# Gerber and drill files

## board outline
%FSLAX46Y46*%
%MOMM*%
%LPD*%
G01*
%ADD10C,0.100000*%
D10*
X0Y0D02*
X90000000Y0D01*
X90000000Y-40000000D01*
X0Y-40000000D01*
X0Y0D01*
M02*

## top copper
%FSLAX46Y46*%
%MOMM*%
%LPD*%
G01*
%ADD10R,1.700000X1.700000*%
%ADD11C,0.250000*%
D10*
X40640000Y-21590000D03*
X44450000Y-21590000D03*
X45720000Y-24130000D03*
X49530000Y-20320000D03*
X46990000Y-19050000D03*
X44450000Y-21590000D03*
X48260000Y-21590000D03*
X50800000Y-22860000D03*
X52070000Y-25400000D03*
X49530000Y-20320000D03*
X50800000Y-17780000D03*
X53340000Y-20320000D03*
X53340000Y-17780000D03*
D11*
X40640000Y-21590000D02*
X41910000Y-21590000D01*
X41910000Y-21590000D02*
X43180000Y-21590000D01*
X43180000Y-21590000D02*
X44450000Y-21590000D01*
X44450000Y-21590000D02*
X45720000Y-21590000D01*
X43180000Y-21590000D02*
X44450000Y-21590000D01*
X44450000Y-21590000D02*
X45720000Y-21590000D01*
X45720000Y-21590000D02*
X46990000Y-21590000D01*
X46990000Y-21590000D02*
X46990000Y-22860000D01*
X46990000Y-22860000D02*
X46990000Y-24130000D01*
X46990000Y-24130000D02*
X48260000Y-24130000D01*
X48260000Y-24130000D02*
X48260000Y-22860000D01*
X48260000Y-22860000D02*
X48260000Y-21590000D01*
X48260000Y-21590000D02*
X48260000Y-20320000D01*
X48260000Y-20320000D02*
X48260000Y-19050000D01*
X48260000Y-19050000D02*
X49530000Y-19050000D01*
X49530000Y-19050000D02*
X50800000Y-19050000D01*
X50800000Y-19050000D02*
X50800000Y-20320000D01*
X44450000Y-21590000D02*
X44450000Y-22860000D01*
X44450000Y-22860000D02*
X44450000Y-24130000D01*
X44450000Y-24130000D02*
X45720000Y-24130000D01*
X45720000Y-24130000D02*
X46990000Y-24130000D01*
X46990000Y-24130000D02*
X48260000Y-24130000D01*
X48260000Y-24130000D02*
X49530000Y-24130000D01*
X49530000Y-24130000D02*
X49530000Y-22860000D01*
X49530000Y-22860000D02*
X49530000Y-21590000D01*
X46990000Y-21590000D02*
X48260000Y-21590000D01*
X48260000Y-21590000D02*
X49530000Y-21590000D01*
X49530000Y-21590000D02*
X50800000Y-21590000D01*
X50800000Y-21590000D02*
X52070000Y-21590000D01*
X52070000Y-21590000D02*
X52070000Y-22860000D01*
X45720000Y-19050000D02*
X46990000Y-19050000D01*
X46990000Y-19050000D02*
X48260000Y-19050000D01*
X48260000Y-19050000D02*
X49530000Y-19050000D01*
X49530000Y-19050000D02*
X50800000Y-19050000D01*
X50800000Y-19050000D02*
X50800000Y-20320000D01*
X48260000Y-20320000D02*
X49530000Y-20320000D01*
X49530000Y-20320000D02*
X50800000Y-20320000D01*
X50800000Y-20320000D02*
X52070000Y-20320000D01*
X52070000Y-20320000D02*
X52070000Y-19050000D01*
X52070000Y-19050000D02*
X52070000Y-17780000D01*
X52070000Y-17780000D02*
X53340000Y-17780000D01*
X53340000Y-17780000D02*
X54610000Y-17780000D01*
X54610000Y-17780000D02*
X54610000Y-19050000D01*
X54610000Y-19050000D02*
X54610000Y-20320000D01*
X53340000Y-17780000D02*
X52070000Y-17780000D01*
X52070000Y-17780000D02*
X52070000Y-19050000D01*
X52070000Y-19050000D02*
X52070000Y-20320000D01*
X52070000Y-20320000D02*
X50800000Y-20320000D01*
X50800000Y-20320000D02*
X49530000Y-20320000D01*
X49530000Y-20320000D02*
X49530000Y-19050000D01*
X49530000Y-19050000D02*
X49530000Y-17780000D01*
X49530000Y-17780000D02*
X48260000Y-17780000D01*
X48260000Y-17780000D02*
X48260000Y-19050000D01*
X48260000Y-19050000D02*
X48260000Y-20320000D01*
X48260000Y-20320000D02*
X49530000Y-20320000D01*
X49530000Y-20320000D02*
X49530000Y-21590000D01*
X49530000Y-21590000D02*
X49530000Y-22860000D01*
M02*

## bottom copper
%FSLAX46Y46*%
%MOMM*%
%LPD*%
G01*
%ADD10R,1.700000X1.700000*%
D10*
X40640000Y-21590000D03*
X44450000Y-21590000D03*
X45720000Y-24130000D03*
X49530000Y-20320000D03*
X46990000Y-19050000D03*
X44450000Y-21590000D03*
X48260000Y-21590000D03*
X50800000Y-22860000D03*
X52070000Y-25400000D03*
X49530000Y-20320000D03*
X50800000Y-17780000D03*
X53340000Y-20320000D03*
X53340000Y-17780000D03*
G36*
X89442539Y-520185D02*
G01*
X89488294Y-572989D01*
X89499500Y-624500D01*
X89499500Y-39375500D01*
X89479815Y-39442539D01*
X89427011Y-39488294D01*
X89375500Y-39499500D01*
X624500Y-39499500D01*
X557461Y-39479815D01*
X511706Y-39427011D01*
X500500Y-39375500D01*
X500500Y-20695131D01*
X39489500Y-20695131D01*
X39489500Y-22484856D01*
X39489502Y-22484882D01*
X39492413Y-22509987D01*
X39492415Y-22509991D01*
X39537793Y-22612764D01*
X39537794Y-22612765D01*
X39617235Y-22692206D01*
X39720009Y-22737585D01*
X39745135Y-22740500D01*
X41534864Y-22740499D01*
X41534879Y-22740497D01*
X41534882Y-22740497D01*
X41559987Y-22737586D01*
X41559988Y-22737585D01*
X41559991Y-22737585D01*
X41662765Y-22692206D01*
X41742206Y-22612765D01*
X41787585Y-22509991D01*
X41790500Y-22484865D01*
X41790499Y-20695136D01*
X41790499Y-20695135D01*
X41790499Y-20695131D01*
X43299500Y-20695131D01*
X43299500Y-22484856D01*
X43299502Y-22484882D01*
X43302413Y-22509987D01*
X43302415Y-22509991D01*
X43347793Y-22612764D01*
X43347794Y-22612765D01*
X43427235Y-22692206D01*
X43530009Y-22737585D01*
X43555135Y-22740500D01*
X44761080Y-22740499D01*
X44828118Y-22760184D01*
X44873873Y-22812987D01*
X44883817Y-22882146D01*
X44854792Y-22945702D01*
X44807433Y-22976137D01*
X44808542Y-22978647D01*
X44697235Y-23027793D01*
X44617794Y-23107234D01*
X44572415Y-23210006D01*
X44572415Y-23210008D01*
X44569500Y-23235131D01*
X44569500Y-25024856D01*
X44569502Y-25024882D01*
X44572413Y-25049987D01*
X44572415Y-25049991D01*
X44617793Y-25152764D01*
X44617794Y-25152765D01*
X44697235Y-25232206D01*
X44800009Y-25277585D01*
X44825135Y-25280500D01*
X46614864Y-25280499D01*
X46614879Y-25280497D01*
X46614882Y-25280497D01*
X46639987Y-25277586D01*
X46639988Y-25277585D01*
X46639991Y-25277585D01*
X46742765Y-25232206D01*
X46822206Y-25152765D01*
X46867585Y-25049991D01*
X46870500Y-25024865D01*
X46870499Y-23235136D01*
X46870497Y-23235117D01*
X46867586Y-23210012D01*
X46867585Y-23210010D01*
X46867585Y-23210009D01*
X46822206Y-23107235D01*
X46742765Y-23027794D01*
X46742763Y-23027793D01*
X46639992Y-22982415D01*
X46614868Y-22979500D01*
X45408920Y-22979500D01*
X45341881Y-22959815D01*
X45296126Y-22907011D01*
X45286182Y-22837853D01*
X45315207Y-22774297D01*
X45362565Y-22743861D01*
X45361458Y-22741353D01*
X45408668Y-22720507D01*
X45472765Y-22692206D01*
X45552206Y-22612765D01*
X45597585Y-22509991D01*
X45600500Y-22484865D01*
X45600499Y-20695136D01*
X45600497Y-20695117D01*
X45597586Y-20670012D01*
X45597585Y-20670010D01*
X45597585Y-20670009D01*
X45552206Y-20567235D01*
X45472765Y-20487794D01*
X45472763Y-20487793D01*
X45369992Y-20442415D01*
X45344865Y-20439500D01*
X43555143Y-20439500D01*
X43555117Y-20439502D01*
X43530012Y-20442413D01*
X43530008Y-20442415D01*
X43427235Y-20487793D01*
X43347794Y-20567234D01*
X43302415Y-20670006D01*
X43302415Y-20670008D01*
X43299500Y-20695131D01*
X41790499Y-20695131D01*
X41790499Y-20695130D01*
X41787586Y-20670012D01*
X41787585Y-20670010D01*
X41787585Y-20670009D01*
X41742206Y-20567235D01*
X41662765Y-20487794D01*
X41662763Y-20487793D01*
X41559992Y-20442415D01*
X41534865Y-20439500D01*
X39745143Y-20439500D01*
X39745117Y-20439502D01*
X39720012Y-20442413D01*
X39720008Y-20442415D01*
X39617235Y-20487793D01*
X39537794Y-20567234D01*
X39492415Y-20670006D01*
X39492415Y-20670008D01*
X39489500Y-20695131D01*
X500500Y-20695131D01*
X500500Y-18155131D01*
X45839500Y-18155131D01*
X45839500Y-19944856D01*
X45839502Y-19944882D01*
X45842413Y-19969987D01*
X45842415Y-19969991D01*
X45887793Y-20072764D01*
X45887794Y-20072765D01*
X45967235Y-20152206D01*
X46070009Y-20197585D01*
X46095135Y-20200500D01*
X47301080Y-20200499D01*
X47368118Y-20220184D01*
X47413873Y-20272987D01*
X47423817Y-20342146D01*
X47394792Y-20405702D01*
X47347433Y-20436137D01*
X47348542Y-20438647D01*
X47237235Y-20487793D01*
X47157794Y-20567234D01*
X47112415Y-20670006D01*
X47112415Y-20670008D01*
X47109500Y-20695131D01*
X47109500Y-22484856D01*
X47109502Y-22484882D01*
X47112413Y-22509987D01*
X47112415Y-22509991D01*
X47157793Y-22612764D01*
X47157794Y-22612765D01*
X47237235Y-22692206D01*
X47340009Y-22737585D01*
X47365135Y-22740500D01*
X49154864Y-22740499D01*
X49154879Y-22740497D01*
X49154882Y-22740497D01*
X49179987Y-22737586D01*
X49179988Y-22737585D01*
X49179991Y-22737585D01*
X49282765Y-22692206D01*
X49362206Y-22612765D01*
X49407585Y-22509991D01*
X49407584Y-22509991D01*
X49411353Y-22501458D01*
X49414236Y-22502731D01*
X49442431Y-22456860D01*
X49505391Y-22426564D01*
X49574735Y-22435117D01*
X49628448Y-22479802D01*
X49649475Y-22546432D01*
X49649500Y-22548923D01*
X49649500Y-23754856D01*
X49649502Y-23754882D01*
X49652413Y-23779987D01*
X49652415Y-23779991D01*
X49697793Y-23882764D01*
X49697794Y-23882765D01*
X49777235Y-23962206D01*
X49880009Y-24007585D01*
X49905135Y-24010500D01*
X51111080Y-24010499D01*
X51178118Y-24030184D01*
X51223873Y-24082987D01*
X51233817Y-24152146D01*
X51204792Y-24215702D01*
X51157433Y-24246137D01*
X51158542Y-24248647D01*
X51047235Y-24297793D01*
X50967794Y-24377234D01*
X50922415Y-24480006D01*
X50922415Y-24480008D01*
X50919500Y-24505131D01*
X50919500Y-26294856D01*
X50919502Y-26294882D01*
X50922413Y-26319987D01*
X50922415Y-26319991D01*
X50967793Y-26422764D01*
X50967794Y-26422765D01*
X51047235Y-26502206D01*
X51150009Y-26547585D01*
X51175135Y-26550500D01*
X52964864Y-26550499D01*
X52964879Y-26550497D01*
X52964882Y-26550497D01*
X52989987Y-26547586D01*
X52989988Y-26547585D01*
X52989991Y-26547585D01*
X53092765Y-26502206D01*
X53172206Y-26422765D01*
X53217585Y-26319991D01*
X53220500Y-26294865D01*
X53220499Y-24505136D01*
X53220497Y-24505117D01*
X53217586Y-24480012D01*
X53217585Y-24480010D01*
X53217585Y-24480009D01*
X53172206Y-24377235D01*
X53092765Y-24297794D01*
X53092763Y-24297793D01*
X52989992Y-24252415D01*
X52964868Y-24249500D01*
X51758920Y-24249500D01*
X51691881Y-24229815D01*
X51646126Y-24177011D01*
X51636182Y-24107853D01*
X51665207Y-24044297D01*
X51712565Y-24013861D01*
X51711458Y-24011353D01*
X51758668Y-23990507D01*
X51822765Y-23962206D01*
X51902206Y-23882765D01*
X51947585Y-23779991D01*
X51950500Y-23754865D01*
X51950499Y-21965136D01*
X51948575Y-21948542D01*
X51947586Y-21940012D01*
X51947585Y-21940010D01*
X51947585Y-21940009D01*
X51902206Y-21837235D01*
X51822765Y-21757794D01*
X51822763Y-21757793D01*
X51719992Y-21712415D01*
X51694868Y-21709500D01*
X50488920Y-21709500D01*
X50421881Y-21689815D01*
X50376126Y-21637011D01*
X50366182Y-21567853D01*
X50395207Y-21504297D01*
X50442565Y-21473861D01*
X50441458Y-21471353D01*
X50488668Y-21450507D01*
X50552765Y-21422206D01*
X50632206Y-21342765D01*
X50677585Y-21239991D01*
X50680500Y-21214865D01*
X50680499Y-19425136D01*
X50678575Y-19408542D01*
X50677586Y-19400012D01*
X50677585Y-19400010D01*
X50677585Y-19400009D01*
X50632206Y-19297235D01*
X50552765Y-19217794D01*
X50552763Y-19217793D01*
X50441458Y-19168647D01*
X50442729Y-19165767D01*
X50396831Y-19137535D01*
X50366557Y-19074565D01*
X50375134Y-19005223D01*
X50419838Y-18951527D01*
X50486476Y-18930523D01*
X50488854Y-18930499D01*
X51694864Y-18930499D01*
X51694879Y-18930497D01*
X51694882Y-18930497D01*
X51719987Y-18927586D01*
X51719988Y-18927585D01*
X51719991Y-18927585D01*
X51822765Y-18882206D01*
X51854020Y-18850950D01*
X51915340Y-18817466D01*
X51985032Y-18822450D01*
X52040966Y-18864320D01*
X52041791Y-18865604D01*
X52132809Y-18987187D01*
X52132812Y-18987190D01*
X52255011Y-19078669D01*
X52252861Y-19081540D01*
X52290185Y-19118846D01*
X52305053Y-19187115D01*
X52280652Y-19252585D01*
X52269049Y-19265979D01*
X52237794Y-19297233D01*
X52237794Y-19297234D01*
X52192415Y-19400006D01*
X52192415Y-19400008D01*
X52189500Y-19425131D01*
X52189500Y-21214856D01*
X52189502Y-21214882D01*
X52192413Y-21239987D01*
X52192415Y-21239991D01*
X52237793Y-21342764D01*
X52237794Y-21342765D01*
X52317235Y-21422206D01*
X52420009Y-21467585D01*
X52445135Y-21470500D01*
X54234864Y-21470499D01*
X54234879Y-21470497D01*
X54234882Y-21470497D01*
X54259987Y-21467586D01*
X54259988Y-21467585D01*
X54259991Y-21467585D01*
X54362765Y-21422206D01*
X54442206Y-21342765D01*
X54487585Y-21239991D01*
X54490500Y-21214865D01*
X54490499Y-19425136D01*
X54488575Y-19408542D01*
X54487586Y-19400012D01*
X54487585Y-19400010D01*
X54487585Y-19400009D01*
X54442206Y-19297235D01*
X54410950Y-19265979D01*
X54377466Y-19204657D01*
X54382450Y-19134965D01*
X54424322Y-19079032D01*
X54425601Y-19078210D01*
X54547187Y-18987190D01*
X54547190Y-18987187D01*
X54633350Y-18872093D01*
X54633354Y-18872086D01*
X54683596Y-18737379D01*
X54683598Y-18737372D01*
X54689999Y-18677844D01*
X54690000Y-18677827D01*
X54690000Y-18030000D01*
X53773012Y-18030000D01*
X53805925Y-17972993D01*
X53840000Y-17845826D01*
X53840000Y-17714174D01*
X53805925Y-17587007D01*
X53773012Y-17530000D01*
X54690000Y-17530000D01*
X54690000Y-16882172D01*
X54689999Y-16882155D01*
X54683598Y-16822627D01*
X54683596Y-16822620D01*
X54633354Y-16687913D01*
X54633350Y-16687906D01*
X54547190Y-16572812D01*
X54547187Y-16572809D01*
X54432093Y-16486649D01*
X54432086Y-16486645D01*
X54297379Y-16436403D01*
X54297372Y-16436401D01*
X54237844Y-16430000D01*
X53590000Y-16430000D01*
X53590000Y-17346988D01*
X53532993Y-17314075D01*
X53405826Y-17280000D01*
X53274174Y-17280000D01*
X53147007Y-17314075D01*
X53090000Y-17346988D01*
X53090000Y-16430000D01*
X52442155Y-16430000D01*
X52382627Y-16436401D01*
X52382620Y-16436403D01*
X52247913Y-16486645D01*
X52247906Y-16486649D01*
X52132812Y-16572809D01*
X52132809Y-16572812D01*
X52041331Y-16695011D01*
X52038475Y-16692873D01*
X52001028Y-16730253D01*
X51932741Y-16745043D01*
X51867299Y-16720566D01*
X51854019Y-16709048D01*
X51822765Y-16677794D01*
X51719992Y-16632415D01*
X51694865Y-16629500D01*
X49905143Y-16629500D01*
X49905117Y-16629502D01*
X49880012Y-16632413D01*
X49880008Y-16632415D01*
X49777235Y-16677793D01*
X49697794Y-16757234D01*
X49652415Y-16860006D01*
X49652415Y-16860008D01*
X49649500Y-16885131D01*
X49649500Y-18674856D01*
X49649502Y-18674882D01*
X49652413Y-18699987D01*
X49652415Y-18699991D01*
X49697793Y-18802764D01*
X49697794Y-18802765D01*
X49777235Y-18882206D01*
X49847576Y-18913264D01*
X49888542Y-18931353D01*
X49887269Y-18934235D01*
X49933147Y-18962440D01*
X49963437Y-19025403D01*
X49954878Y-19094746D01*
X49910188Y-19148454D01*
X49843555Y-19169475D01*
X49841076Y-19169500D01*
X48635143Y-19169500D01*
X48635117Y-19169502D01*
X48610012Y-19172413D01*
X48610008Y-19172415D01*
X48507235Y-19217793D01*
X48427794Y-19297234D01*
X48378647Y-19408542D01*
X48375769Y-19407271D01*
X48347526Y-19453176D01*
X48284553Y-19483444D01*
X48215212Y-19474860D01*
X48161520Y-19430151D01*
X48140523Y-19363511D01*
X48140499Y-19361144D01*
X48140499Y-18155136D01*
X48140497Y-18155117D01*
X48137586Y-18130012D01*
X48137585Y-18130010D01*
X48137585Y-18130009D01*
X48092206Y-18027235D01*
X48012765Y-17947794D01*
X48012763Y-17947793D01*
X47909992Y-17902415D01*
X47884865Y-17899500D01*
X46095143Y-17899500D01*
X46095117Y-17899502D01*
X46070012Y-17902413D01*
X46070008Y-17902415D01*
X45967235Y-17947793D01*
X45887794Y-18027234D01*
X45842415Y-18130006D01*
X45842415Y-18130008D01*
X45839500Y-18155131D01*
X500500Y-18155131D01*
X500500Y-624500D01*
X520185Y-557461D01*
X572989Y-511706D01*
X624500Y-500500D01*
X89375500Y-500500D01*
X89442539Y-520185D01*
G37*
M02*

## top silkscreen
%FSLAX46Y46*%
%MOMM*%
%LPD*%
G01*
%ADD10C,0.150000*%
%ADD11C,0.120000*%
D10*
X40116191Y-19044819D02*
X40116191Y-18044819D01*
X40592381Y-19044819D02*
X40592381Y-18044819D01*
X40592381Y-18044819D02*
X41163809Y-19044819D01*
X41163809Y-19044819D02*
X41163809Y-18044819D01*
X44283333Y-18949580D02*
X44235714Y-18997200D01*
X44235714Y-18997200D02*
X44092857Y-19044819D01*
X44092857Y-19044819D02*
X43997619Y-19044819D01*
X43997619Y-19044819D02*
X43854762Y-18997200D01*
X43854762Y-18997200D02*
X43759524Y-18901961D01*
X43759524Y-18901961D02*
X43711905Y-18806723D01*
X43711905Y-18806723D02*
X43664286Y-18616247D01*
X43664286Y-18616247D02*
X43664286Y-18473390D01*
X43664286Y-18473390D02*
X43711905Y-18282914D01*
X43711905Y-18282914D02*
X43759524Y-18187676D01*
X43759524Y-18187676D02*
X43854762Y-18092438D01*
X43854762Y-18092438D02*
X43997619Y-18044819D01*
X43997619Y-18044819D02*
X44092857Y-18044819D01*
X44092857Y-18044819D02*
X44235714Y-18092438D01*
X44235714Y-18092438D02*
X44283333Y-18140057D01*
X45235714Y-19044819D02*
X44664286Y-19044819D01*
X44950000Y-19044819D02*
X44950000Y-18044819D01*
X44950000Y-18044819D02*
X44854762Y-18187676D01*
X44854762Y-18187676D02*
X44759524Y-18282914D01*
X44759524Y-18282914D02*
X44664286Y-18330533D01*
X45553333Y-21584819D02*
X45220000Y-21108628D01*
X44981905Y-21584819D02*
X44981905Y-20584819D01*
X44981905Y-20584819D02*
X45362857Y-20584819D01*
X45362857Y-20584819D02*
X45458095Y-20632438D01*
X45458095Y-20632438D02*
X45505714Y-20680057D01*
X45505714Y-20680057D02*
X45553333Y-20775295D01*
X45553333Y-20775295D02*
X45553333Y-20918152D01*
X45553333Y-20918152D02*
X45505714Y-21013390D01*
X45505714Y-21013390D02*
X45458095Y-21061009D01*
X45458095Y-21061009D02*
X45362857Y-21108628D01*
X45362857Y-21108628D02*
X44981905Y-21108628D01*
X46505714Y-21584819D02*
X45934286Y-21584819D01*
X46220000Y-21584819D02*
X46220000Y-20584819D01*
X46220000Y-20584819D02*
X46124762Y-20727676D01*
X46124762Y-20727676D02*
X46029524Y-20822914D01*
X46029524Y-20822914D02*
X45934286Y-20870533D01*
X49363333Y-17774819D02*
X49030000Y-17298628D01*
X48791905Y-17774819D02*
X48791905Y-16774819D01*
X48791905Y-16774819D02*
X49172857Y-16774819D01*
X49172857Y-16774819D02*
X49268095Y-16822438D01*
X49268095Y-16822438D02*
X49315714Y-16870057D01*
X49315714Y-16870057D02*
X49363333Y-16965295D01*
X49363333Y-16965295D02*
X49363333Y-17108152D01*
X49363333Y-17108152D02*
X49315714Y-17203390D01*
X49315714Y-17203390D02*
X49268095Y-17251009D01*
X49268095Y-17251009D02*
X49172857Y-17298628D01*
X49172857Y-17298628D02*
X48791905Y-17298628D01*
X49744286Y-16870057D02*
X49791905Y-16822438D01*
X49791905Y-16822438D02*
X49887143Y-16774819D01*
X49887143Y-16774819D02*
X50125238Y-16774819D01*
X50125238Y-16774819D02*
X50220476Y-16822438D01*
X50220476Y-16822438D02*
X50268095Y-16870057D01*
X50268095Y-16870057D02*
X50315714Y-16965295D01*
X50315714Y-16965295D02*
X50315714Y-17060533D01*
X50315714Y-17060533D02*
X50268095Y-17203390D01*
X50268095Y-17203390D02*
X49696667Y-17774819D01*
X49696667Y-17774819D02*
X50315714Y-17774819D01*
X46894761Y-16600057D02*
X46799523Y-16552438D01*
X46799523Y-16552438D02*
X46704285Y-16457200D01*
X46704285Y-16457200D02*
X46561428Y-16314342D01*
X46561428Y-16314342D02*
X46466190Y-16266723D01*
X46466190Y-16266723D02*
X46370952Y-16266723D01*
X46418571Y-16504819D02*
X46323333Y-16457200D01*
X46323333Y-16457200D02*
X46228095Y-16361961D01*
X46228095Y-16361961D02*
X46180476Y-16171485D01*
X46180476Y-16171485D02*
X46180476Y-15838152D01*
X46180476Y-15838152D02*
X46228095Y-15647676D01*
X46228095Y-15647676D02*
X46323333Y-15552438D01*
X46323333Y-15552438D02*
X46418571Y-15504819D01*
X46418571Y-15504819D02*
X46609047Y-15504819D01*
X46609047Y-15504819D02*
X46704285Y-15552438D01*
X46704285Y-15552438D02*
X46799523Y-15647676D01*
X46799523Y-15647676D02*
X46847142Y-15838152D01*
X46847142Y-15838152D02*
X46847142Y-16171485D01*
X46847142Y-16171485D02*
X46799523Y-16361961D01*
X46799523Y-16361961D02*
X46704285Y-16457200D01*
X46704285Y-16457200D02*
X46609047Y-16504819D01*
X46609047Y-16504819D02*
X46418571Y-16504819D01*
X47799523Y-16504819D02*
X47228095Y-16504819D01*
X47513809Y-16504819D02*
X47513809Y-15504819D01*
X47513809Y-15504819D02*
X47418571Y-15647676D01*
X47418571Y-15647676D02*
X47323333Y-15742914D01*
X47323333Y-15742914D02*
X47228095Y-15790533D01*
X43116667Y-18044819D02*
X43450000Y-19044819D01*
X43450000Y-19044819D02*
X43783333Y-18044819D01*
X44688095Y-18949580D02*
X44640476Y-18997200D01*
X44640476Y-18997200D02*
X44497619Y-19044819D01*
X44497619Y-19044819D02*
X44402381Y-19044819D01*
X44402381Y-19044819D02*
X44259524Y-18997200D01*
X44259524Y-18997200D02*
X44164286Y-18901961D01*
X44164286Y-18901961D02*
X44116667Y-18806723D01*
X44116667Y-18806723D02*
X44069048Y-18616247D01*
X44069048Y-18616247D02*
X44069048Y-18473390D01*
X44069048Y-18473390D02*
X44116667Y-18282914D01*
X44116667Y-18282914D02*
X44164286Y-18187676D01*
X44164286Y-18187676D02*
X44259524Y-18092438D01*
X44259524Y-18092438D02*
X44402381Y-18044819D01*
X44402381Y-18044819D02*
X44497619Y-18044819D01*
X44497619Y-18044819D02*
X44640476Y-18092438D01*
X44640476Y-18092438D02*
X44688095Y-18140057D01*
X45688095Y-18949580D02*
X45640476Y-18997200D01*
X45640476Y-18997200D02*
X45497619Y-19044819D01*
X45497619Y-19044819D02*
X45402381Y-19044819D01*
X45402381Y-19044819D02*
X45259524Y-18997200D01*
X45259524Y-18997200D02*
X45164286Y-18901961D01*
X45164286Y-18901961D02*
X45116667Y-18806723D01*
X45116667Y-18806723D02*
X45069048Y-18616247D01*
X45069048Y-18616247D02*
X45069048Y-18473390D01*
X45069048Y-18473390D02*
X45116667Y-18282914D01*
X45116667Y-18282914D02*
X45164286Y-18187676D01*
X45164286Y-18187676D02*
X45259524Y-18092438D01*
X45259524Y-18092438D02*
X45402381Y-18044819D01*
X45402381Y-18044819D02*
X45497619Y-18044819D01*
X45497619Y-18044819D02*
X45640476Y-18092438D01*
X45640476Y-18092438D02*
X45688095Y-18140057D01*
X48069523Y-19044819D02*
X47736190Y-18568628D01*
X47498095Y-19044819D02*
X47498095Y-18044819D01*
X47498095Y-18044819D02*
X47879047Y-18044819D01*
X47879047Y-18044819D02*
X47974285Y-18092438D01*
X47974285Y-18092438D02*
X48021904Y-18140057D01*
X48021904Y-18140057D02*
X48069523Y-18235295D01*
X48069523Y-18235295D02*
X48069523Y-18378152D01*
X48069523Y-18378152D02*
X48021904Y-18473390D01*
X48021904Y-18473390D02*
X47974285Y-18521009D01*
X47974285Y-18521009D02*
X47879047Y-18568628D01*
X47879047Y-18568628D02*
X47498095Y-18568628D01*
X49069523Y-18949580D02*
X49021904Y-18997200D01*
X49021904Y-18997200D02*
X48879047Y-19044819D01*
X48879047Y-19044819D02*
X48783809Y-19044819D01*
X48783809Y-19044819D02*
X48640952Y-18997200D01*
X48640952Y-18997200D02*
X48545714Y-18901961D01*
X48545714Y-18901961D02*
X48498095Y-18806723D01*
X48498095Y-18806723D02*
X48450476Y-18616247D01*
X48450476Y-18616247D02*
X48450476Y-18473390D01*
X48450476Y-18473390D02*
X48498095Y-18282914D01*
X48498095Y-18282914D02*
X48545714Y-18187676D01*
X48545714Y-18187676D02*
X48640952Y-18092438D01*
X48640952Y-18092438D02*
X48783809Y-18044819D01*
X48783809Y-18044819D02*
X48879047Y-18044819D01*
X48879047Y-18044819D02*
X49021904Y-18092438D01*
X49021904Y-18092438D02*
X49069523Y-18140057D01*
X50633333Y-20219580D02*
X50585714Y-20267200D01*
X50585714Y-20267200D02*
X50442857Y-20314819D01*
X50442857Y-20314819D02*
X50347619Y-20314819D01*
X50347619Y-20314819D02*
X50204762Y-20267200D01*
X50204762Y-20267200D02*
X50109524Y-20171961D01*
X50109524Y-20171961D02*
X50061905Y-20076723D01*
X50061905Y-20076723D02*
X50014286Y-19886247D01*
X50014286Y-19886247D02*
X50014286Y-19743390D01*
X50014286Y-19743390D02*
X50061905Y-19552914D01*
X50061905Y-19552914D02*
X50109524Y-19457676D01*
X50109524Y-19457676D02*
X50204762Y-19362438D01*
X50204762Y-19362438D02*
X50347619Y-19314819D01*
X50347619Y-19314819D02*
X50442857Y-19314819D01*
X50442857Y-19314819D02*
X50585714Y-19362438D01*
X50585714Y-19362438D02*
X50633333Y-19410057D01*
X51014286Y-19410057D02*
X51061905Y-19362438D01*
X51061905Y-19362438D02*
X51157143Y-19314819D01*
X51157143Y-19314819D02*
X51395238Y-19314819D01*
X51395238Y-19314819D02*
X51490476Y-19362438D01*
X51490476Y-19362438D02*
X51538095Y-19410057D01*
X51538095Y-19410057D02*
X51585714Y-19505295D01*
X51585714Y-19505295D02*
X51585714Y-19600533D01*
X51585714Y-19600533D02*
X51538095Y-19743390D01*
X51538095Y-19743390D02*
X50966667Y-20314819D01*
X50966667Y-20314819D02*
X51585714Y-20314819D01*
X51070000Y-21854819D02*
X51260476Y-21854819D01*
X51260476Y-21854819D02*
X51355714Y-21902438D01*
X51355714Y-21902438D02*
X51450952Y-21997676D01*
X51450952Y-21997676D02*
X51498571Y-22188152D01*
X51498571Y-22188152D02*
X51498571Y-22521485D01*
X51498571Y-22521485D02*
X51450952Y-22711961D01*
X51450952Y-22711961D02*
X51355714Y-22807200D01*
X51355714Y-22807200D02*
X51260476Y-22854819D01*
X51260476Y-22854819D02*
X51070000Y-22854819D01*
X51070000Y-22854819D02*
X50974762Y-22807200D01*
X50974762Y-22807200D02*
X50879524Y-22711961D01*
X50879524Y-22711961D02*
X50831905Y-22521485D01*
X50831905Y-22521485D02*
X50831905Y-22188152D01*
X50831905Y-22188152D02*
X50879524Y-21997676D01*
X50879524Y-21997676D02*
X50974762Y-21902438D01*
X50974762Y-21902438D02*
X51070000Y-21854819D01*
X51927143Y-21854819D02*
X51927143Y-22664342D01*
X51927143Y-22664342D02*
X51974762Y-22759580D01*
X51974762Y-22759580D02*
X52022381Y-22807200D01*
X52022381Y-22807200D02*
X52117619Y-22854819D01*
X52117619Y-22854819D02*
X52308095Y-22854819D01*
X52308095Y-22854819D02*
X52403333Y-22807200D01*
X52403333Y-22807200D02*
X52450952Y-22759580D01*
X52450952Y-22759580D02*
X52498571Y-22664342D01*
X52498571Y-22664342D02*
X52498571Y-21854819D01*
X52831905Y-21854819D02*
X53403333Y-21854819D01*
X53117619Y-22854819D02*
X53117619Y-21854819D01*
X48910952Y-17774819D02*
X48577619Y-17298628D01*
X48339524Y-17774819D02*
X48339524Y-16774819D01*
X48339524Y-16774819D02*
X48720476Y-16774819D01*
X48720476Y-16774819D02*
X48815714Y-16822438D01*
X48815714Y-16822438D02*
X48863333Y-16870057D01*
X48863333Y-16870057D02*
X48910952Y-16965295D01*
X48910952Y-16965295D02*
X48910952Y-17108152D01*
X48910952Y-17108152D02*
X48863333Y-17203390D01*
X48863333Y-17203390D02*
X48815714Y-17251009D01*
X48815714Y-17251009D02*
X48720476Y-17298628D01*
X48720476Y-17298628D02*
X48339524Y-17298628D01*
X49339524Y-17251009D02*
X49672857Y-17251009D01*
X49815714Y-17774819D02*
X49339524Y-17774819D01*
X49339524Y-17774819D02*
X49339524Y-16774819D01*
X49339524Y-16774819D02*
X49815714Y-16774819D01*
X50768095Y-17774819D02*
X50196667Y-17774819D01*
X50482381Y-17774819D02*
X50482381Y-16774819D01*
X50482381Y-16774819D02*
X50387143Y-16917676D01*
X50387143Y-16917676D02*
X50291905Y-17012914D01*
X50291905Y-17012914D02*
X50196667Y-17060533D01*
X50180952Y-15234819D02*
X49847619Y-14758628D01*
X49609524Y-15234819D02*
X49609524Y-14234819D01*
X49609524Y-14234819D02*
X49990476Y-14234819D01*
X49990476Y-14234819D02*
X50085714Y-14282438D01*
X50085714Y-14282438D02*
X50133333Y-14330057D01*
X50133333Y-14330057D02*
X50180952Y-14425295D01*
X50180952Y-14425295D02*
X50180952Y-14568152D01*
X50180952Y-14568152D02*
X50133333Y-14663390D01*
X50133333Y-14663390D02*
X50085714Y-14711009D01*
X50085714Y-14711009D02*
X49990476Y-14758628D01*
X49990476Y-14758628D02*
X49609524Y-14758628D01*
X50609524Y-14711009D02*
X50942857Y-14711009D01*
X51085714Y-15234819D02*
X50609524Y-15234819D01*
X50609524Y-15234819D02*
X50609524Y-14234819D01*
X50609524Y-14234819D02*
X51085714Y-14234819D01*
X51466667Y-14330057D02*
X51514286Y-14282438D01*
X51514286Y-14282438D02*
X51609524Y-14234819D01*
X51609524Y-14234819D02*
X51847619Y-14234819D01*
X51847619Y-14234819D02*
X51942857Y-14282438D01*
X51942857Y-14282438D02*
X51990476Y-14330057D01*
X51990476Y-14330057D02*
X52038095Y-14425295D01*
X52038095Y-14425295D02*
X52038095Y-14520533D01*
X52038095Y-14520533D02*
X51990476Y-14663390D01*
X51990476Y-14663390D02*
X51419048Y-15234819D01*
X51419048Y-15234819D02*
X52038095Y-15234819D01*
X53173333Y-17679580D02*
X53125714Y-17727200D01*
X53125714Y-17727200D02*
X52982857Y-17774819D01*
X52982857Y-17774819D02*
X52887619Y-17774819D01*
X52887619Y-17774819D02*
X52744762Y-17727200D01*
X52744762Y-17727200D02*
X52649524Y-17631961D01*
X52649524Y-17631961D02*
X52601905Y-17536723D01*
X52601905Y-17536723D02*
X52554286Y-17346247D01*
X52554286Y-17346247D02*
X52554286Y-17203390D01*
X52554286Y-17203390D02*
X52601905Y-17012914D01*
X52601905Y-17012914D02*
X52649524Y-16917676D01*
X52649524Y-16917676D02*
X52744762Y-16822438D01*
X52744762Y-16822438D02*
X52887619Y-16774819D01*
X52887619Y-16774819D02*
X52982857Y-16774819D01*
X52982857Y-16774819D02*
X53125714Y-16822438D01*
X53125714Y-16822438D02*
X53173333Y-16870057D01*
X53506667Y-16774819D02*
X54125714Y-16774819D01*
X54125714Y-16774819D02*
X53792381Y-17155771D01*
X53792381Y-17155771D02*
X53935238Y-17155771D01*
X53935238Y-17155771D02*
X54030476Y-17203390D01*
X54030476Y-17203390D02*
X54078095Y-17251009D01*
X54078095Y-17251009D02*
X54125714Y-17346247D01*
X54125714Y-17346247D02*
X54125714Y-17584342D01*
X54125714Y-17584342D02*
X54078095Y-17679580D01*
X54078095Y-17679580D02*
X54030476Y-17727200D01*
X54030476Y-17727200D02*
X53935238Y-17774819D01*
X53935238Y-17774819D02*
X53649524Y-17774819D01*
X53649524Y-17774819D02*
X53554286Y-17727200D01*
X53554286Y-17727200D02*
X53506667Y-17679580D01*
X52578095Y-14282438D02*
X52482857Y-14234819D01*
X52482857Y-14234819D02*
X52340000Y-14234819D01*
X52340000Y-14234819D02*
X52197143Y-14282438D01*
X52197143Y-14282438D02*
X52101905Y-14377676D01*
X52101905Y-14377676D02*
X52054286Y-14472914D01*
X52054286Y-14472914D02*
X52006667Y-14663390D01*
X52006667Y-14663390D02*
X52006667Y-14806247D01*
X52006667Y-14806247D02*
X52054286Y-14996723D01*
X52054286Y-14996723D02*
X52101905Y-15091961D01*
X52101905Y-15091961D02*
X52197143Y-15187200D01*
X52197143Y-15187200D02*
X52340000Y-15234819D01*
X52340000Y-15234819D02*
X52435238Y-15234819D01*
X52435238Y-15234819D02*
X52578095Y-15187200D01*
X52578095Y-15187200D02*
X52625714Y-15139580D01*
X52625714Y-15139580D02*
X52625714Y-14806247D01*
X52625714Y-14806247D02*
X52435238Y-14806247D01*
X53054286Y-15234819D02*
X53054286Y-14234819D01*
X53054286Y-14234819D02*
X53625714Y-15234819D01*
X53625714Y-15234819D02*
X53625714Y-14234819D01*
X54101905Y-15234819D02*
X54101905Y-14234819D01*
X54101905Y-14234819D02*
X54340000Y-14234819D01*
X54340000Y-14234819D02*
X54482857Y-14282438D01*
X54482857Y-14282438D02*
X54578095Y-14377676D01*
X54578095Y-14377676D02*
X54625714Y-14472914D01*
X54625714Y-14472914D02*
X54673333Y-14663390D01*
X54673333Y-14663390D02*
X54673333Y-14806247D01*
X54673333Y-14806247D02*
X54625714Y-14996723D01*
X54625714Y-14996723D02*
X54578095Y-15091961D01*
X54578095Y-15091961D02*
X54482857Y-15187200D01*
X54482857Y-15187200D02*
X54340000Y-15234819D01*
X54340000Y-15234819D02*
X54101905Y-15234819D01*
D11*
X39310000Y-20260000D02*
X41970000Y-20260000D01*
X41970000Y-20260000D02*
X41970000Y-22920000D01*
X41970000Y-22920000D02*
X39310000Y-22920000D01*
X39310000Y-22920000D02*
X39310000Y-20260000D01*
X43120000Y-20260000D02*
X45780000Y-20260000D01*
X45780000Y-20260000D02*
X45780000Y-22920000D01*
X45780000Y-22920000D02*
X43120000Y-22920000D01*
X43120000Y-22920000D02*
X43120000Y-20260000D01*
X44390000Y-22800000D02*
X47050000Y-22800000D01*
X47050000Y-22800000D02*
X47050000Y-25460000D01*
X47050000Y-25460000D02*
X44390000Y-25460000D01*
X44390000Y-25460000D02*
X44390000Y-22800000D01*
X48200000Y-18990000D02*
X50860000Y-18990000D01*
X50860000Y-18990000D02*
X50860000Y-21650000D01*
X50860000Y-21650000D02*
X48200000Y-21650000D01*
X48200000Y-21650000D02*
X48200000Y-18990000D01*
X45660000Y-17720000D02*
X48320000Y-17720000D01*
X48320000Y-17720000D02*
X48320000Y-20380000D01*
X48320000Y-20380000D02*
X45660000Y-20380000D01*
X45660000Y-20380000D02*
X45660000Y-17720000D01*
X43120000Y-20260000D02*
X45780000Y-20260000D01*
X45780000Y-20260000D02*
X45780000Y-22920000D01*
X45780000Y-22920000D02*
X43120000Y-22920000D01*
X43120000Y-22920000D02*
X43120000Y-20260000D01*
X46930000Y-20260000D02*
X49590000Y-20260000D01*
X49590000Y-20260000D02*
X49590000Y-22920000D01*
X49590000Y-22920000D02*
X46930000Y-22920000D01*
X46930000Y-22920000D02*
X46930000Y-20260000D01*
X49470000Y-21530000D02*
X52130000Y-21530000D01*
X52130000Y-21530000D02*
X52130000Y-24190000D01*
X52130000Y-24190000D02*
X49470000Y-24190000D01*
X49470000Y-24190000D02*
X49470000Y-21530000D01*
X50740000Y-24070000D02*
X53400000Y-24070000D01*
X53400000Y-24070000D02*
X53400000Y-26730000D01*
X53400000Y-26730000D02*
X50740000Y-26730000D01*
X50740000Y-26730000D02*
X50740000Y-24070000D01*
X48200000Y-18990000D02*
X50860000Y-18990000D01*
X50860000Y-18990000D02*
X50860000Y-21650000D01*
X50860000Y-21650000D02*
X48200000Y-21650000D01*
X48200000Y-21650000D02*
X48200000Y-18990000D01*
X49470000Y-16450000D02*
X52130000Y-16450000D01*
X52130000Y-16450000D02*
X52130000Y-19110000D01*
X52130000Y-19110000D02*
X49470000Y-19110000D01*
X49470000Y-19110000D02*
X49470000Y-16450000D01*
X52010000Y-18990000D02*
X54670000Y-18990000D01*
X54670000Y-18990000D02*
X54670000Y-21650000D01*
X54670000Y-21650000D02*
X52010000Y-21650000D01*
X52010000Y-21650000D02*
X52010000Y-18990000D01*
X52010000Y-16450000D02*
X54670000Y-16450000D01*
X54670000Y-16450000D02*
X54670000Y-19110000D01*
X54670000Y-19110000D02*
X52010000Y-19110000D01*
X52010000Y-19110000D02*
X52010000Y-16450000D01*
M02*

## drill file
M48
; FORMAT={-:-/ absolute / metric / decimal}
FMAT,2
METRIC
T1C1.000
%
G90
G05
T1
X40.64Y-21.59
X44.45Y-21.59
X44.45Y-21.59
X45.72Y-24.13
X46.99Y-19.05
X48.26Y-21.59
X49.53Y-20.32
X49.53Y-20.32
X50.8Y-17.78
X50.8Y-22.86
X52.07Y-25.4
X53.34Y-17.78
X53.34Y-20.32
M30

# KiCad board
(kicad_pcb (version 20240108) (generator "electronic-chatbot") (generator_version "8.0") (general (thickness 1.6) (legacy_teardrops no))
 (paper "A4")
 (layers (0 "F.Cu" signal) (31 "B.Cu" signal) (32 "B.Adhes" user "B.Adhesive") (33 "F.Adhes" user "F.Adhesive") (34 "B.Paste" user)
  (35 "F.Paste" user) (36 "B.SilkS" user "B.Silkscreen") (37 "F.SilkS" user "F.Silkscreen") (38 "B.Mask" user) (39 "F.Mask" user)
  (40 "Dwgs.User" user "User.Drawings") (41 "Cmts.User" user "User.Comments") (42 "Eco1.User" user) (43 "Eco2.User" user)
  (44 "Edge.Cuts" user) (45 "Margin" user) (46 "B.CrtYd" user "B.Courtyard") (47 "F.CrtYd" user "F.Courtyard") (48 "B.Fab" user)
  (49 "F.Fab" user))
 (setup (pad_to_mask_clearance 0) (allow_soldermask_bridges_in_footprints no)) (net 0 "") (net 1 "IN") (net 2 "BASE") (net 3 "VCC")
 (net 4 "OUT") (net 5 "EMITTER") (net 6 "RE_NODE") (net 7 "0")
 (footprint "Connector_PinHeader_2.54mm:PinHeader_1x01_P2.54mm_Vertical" (layer "F.Cu") (at 40.64 21.59)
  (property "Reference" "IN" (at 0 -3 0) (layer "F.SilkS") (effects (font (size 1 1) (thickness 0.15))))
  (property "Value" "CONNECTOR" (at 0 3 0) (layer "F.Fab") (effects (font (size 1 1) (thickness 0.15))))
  (fp_line (start -1.33 -1.33) (end 1.33 -1.33) (stroke (width 0.12) (type solid)) (layer "F.SilkS"))
  (fp_line (start 1.33 -1.33) (end 1.33 1.33) (stroke (width 0.12) (type solid)) (layer "F.SilkS"))
  (fp_line (start 1.33 1.33) (end -1.33 1.33) (stroke (width 0.12) (type solid)) (layer "F.SilkS"))
  (fp_line (start -1.33 1.33) (end -1.33 -1.33) (stroke (width 0.12) (type solid)) (layer "F.SilkS"))
  (pad "1" thru_hole rect (at 0 0) (size 1.7 1.7) (drill 1.0) (layers "*.Cu" "*.Mask") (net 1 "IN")))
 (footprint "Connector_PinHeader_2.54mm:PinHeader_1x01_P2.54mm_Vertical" (layer "F.Cu") (at 44.45 21.59)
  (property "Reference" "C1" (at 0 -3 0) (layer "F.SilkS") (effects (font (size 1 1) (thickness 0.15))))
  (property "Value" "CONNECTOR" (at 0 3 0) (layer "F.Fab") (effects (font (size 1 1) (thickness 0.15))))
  (fp_line (start -1.33 -1.33) (end 1.33 -1.33) (stroke (width 0.12) (type solid)) (layer "F.SilkS"))
  (fp_line (start 1.33 -1.33) (end 1.33 1.33) (stroke (width 0.12) (type solid)) (layer "F.SilkS"))
  (fp_line (start 1.33 1.33) (end -1.33 1.33) (stroke (width 0.12) (type solid)) (layer "F.SilkS"))
  (fp_line (start -1.33 1.33) (end -1.33 -1.33) (stroke (width 0.12) (type solid)) (layer "F.SilkS"))
  (pad "1" thru_hole rect (at 0 0) (size 1.7 1.7) (drill 1.0) (layers "*.Cu" "*.Mask") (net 1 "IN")))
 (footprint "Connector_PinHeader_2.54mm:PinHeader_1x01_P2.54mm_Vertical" (layer "F.Cu") (at 45.72 24.13)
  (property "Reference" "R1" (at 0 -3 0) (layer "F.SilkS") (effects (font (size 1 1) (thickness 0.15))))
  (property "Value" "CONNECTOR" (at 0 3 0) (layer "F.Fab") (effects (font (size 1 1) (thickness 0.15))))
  (fp_line (start -1.33 -1.33) (end 1.33 -1.33) (stroke (width 0.12) (type solid)) (layer "F.SilkS"))
  (fp_line (start 1.33 -1.33) (end 1.33 1.33) (stroke (width 0.12) (type solid)) (layer "F.SilkS"))
  (fp_line (start 1.33 1.33) (end -1.33 1.33) (stroke (width 0.12) (type solid)) (layer "F.SilkS"))
  (fp_line (start -1.33 1.33) (end -1.33 -1.33) (stroke (width 0.12) (type solid)) (layer "F.SilkS"))
  (pad "1" thru_hole rect (at 0 0) (size 1.7 1.7) (drill 1.0) (layers "*.Cu" "*.Mask") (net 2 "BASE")))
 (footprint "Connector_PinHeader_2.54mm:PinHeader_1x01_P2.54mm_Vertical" (layer "F.Cu") (at 49.53 20.32)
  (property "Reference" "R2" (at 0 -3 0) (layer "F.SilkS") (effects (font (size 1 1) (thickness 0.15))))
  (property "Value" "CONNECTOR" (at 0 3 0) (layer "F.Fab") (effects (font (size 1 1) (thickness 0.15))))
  (fp_line (start -1.33 -1.33) (end 1.33 -1.33) (stroke (width 0.12) (type solid)) (layer "F.SilkS"))
  (fp_line (start 1.33 -1.33) (end 1.33 1.33) (stroke (width 0.12) (type solid)) (layer "F.SilkS"))
  (fp_line (start 1.33 1.33) (end -1.33 1.33) (stroke (width 0.12) (type solid)) (layer "F.SilkS"))
  (fp_line (start -1.33 1.33) (end -1.33 -1.33) (stroke (width 0.12) (type solid)) (layer "F.SilkS"))
  (pad "1" thru_hole rect (at 0 0) (size 1.7 1.7) (drill 1.0) (layers "*.Cu" "*.Mask") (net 2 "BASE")))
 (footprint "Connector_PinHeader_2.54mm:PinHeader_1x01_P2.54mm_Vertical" (layer "F.Cu") (at 46.99 19.05)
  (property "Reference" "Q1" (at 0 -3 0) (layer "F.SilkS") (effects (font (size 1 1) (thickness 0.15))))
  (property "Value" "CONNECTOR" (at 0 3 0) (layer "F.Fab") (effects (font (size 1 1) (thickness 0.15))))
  (fp_line (start -1.33 -1.33) (end 1.33 -1.33) (stroke (width 0.12) (type solid)) (layer "F.SilkS"))
  (fp_line (start 1.33 -1.33) (end 1.33 1.33) (stroke (width 0.12) (type solid)) (layer "F.SilkS"))
  (fp_line (start 1.33 1.33) (end -1.33 1.33) (stroke (width 0.12) (type solid)) (layer "F.SilkS"))
  (fp_line (start -1.33 1.33) (end -1.33 -1.33) (stroke (width 0.12) (type solid)) (layer "F.SilkS"))
  (pad "1" thru_hole rect (at 0 0) (size 1.7 1.7) (drill 1.0) (layers "*.Cu" "*.Mask") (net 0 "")))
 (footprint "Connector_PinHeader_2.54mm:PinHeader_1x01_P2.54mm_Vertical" (layer "F.Cu") (at 44.45 21.59)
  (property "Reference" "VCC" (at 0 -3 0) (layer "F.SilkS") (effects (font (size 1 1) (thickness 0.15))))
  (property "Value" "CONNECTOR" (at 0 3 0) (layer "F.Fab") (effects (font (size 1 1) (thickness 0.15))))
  (fp_line (start -1.33 -1.33) (end 1.33 -1.33) (stroke (width 0.12) (type solid)) (layer "F.SilkS"))
  (fp_line (start 1.33 -1.33) (end 1.33 1.33) (stroke (width 0.12) (type solid)) (layer "F.SilkS"))
  (fp_line (start 1.33 1.33) (end -1.33 1.33) (stroke (width 0.12) (type solid)) (layer "F.SilkS"))
  (fp_line (start -1.33 1.33) (end -1.33 -1.33) (stroke (width 0.12) (type solid)) (layer "F.SilkS"))
  (pad "1" thru_hole rect (at 0 0) (size 1.7 1.7) (drill 1.0) (layers "*.Cu" "*.Mask") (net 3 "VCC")))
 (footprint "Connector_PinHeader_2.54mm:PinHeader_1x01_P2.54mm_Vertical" (layer "F.Cu") (at 48.26 21.59)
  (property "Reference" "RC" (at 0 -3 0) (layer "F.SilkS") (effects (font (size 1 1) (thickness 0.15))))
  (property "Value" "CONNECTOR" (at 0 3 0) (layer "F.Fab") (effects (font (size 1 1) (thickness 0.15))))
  (fp_line (start -1.33 -1.33) (end 1.33 -1.33) (stroke (width 0.12) (type solid)) (layer "F.SilkS"))
  (fp_line (start 1.33 -1.33) (end 1.33 1.33) (stroke (width 0.12) (type solid)) (layer "F.SilkS"))
  (fp_line (start 1.33 1.33) (end -1.33 1.33) (stroke (width 0.12) (type solid)) (layer "F.SilkS"))
  (fp_line (start -1.33 1.33) (end -1.33 -1.33) (stroke (width 0.12) (type solid)) (layer "F.SilkS"))
  (pad "1" thru_hole rect (at 0 0) (size 1.7 1.7) (drill 1.0) (layers "*.Cu" "*.Mask") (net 3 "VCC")))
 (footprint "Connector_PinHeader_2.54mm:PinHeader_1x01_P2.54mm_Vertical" (layer "F.Cu") (at 50.8 22.86)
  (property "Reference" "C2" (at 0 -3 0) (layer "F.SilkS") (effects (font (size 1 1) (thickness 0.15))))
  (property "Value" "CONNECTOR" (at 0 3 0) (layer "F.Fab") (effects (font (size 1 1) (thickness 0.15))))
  (fp_line (start -1.33 -1.33) (end 1.33 -1.33) (stroke (width 0.12) (type solid)) (layer "F.SilkS"))
  (fp_line (start 1.33 -1.33) (end 1.33 1.33) (stroke (width 0.12) (type solid)) (layer "F.SilkS"))
  (fp_line (start 1.33 1.33) (end -1.33 1.33) (stroke (width 0.12) (type solid)) (layer "F.SilkS"))
  (fp_line (start -1.33 1.33) (end -1.33 -1.33) (stroke (width 0.12) (type solid)) (layer "F.SilkS"))
  (pad "1" thru_hole rect (at 0 0) (size 1.7 1.7) (drill 1.0) (layers "*.Cu" "*.Mask") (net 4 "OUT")))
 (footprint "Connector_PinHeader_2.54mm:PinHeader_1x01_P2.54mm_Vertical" (layer "F.Cu") (at 52.07 25.4)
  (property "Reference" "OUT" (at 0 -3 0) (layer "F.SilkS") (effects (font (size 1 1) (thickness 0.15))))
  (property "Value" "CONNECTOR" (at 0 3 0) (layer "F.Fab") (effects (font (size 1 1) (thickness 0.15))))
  (fp_line (start -1.33 -1.33) (end 1.33 -1.33) (stroke (width 0.12) (type solid)) (layer "F.SilkS"))
  (fp_line (start 1.33 -1.33) (end 1.33 1.33) (stroke (width 0.12) (type solid)) (layer "F.SilkS"))
  (fp_line (start 1.33 1.33) (end -1.33 1.33) (stroke (width 0.12) (type solid)) (layer "F.SilkS"))
  (fp_line (start -1.33 1.33) (end -1.33 -1.33) (stroke (width 0.12) (type solid)) (layer "F.SilkS"))
  (pad "1" thru_hole rect (at 0 0) (size 1.7 1.7) (drill 1.0) (layers "*.Cu" "*.Mask") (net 4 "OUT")))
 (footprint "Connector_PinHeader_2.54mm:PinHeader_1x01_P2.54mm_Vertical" (layer "F.Cu") (at 49.53 20.32)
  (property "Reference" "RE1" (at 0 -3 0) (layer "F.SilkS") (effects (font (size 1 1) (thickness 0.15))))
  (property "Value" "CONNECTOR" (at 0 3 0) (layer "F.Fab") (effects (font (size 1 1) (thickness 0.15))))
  (fp_line (start -1.33 -1.33) (end 1.33 -1.33) (stroke (width 0.12) (type solid)) (layer "F.SilkS"))
  (fp_line (start 1.33 -1.33) (end 1.33 1.33) (stroke (width 0.12) (type solid)) (layer "F.SilkS"))
  (fp_line (start 1.33 1.33) (end -1.33 1.33) (stroke (width 0.12) (type solid)) (layer "F.SilkS"))
  (fp_line (start -1.33 1.33) (end -1.33 -1.33) (stroke (width 0.12) (type solid)) (layer "F.SilkS"))
  (pad "1" thru_hole rect (at 0 0) (size 1.7 1.7) (drill 1.0) (layers "*.Cu" "*.Mask") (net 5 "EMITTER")))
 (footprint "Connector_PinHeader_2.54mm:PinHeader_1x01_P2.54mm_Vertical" (layer "F.Cu") (at 50.8 17.78)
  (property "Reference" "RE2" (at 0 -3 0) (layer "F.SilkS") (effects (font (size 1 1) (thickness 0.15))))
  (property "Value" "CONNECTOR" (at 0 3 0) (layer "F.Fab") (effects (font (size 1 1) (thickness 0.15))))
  (fp_line (start -1.33 -1.33) (end 1.33 -1.33) (stroke (width 0.12) (type solid)) (layer "F.SilkS"))
  (fp_line (start 1.33 -1.33) (end 1.33 1.33) (stroke (width 0.12) (type solid)) (layer "F.SilkS"))
  (fp_line (start 1.33 1.33) (end -1.33 1.33) (stroke (width 0.12) (type solid)) (layer "F.SilkS"))
  (fp_line (start -1.33 1.33) (end -1.33 -1.33) (stroke (width 0.12) (type solid)) (layer "F.SilkS"))
  (pad "1" thru_hole rect (at 0 0) (size 1.7 1.7) (drill 1.0) (layers "*.Cu" "*.Mask") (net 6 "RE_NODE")))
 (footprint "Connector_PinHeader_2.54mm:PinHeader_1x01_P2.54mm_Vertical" (layer "F.Cu") (at 53.34 20.32)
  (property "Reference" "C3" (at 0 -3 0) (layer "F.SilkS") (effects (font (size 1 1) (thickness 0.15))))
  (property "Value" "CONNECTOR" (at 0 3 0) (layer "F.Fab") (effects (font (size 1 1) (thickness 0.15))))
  (fp_line (start -1.33 -1.33) (end 1.33 -1.33) (stroke (width 0.12) (type solid)) (layer "F.SilkS"))
  (fp_line (start 1.33 -1.33) (end 1.33 1.33) (stroke (width 0.12) (type solid)) (layer "F.SilkS"))
  (fp_line (start 1.33 1.33) (end -1.33 1.33) (stroke (width 0.12) (type solid)) (layer "F.SilkS"))
  (fp_line (start -1.33 1.33) (end -1.33 -1.33) (stroke (width 0.12) (type solid)) (layer "F.SilkS"))
  (pad "1" thru_hole rect (at 0 0) (size 1.7 1.7) (drill 1.0) (layers "*.Cu" "*.Mask") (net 6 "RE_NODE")))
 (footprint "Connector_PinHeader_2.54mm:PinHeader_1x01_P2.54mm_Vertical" (layer "F.Cu") (at 53.34 17.78)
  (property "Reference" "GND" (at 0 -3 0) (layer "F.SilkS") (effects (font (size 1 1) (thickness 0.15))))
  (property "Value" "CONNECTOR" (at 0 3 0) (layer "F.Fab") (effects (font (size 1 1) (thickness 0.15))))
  (fp_line (start -1.33 -1.33) (end 1.33 -1.33) (stroke (width 0.12) (type solid)) (layer "F.SilkS"))
  (fp_line (start 1.33 -1.33) (end 1.33 1.33) (stroke (width 0.12) (type solid)) (layer "F.SilkS"))
  (fp_line (start 1.33 1.33) (end -1.33 1.33) (stroke (width 0.12) (type solid)) (layer "F.SilkS"))
  (fp_line (start -1.33 1.33) (end -1.33 -1.33) (stroke (width 0.12) (type solid)) (layer "F.SilkS"))
  (pad "1" thru_hole rect (at 0 0) (size 1.7 1.7) (drill 1.0) (layers "*.Cu" "*.Mask") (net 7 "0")))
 (gr_rect (start 0 0) (end 90.0 40.0) (layer "Edge.Cuts") (stroke (width 0.1) (type solid)) (fill none))
 (segment (start 40.64 21.59) (end 41.91 21.59) (width 0.25) (layer "F.Cu") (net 1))
 (segment (start 41.91 21.59) (end 43.18 21.59) (width 0.25) (layer "F.Cu") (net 1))
 (segment (start 43.18 21.59) (end 44.45 21.59) (width 0.25) (layer "F.Cu") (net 1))
 (segment (start 44.45 21.59) (end 45.72 21.59) (width 0.25) (layer "F.Cu") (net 1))
 (segment (start 43.18 21.59) (end 44.45 21.59) (width 0.25) (layer "F.Cu") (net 2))
 (segment (start 44.45 21.59) (end 45.72 21.59) (width 0.25) (layer "F.Cu") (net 2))
 (segment (start 45.72 21.59) (end 46.99 21.59) (width 0.25) (layer "F.Cu") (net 2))
 (segment (start 46.99 21.59) (end 46.99 22.86) (width 0.25) (layer "F.Cu") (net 2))
 (segment (start 46.99 22.86) (end 46.99 24.13) (width 0.25) (layer "F.Cu") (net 2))
 (segment (start 46.99 24.13) (end 48.26 24.13) (width 0.25) (layer "F.Cu") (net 2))
 (segment (start 48.26 24.13) (end 48.26 22.86) (width 0.25) (layer "F.Cu") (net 2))
 (segment (start 48.26 22.86) (end 48.26 21.59) (width 0.25) (layer "F.Cu") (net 2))
 (segment (start 48.26 21.59) (end 48.26 20.32) (width 0.25) (layer "F.Cu") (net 2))
 (segment (start 48.26 20.32) (end 48.26 19.05) (width 0.25) (layer "F.Cu") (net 2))
 (segment (start 48.26 19.05) (end 49.53 19.05) (width 0.25) (layer "F.Cu") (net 2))
 (segment (start 49.53 19.05) (end 50.8 19.05) (width 0.25) (layer "F.Cu") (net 2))
 (segment (start 50.8 19.05) (end 50.8 20.32) (width 0.25) (layer "F.Cu") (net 2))
 (segment (start 44.45 21.59) (end 44.45 22.86) (width 0.25) (layer "F.Cu") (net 3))
 (segment (start 44.45 22.86) (end 44.45 24.13) (width 0.25) (layer "F.Cu") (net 3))
 (segment (start 44.45 24.13) (end 45.72 24.13) (width 0.25) (layer "F.Cu") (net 3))
 (segment (start 45.72 24.13) (end 46.99 24.13) (width 0.25) (layer "F.Cu") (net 3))
 (segment (start 46.99 24.13) (end 48.26 24.13) (width 0.25) (layer "F.Cu") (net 3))
 (segment (start 48.26 24.13) (end 49.53 24.13) (width 0.25) (layer "F.Cu") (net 3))
 (segment (start 49.53 24.13) (end 49.53 22.86) (width 0.25) (layer "F.Cu") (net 3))
 (segment (start 49.53 22.86) (end 49.53 21.59) (width 0.25) (layer "F.Cu") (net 3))
 (segment (start 46.99 21.59) (end 48.26 21.59) (width 0.25) (layer "F.Cu") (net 4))
 (segment (start 48.26 21.59) (end 49.53 21.59) (width 0.25) (layer "F.Cu") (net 4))
 (segment (start 49.53 21.59) (end 50.8 21.59) (width 0.25) (layer "F.Cu") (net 4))
 (segment (start 50.8 21.59) (end 52.07 21.59) (width 0.25) (layer "F.Cu") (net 4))
 (segment (start 52.07 21.59) (end 52.07 22.86) (width 0.25) (layer "F.Cu") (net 4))
 (segment (start 45.72 19.05) (end 46.99 19.05) (width 0.25) (layer "F.Cu") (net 5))
 (segment (start 46.99 19.05) (end 48.26 19.05) (width 0.25) (layer "F.Cu") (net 5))
 (segment (start 48.26 19.05) (end 49.53 19.05) (width 0.25) (layer "F.Cu") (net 5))
 (segment (start 49.53 19.05) (end 50.8 19.05) (width 0.25) (layer "F.Cu") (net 5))
 (segment (start 50.8 19.05) (end 50.8 20.32) (width 0.25) (layer "F.Cu") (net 5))
 (segment (start 48.26 20.32) (end 49.53 20.32) (width 0.25) (layer "F.Cu") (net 6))
 (segment (start 49.53 20.32) (end 50.8 20.32) (width 0.25) (layer "F.Cu") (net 6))
 (segment (start 50.8 20.32) (end 52.07 20.32) (width 0.25) (layer "F.Cu") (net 6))
 (segment (start 52.07 20.32) (end 52.07 19.05) (width 0.25) (layer "F.Cu") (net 6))
 (segment (start 52.07 19.05) (end 52.07 17.78) (width 0.25) (layer "F.Cu") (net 6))
 (segment (start 52.07 17.78) (end 53.34 17.78) (width 0.25) (layer "F.Cu") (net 6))
 (segment (start 53.34 17.78) (end 54.61 17.78) (width 0.25) (layer "F.Cu") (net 6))
 (segment (start 54.61 17.78) (end 54.61 19.05) (width 0.25) (layer "F.Cu") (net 6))
 (segment (start 54.61 19.05) (end 54.61 20.32) (width 0.25) (layer "F.Cu") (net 6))
 (segment (start 53.34 17.78) (end 52.07 17.78) (width 0.25) (layer "F.Cu") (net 7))
 (segment (start 52.07 17.78) (end 52.07 19.05) (width 0.25) (layer "F.Cu") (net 7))
 (segment (start 52.07 19.05) (end 52.07 20.32) (width 0.25) (layer "F.Cu") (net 7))
 (segment (start 52.07 20.32) (end 50.8 20.32) (width 0.25) (layer "F.Cu") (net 7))
 (segment (start 50.8 20.32) (end 49.53 20.32) (width 0.25) (layer "F.Cu") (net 7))
 (segment (start 49.53 20.32) (end 49.53 19.05) (width 0.25) (layer "F.Cu") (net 7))
 (segment (start 49.53 19.05) (end 49.53 17.78) (width 0.25) (layer "F.Cu") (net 7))
 (segment (start 49.53 17.78) (end 48.26 17.78) (width 0.25) (layer "F.Cu") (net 7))
 (segment (start 48.26 17.78) (end 48.26 19.05) (width 0.25) (layer "F.Cu") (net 7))
 (segment (start 48.26 19.05) (end 48.26 20.32) (width 0.25) (layer "F.Cu") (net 7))
 (segment (start 48.26 20.32) (end 49.53 20.32) (width 0.25) (layer "F.Cu") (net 7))
 (segment (start 49.53 20.32) (end 49.53 21.59) (width 0.25) (layer "F.Cu") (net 7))
 (segment (start 49.53 21.59) (end 49.53 22.86) (width 0.25) (layer "F.Cu") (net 7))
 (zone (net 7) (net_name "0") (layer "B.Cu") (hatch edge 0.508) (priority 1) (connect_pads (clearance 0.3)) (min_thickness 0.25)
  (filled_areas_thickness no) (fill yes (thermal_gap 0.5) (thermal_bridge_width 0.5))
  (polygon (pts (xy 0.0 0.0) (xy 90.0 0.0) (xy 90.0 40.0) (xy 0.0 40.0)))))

